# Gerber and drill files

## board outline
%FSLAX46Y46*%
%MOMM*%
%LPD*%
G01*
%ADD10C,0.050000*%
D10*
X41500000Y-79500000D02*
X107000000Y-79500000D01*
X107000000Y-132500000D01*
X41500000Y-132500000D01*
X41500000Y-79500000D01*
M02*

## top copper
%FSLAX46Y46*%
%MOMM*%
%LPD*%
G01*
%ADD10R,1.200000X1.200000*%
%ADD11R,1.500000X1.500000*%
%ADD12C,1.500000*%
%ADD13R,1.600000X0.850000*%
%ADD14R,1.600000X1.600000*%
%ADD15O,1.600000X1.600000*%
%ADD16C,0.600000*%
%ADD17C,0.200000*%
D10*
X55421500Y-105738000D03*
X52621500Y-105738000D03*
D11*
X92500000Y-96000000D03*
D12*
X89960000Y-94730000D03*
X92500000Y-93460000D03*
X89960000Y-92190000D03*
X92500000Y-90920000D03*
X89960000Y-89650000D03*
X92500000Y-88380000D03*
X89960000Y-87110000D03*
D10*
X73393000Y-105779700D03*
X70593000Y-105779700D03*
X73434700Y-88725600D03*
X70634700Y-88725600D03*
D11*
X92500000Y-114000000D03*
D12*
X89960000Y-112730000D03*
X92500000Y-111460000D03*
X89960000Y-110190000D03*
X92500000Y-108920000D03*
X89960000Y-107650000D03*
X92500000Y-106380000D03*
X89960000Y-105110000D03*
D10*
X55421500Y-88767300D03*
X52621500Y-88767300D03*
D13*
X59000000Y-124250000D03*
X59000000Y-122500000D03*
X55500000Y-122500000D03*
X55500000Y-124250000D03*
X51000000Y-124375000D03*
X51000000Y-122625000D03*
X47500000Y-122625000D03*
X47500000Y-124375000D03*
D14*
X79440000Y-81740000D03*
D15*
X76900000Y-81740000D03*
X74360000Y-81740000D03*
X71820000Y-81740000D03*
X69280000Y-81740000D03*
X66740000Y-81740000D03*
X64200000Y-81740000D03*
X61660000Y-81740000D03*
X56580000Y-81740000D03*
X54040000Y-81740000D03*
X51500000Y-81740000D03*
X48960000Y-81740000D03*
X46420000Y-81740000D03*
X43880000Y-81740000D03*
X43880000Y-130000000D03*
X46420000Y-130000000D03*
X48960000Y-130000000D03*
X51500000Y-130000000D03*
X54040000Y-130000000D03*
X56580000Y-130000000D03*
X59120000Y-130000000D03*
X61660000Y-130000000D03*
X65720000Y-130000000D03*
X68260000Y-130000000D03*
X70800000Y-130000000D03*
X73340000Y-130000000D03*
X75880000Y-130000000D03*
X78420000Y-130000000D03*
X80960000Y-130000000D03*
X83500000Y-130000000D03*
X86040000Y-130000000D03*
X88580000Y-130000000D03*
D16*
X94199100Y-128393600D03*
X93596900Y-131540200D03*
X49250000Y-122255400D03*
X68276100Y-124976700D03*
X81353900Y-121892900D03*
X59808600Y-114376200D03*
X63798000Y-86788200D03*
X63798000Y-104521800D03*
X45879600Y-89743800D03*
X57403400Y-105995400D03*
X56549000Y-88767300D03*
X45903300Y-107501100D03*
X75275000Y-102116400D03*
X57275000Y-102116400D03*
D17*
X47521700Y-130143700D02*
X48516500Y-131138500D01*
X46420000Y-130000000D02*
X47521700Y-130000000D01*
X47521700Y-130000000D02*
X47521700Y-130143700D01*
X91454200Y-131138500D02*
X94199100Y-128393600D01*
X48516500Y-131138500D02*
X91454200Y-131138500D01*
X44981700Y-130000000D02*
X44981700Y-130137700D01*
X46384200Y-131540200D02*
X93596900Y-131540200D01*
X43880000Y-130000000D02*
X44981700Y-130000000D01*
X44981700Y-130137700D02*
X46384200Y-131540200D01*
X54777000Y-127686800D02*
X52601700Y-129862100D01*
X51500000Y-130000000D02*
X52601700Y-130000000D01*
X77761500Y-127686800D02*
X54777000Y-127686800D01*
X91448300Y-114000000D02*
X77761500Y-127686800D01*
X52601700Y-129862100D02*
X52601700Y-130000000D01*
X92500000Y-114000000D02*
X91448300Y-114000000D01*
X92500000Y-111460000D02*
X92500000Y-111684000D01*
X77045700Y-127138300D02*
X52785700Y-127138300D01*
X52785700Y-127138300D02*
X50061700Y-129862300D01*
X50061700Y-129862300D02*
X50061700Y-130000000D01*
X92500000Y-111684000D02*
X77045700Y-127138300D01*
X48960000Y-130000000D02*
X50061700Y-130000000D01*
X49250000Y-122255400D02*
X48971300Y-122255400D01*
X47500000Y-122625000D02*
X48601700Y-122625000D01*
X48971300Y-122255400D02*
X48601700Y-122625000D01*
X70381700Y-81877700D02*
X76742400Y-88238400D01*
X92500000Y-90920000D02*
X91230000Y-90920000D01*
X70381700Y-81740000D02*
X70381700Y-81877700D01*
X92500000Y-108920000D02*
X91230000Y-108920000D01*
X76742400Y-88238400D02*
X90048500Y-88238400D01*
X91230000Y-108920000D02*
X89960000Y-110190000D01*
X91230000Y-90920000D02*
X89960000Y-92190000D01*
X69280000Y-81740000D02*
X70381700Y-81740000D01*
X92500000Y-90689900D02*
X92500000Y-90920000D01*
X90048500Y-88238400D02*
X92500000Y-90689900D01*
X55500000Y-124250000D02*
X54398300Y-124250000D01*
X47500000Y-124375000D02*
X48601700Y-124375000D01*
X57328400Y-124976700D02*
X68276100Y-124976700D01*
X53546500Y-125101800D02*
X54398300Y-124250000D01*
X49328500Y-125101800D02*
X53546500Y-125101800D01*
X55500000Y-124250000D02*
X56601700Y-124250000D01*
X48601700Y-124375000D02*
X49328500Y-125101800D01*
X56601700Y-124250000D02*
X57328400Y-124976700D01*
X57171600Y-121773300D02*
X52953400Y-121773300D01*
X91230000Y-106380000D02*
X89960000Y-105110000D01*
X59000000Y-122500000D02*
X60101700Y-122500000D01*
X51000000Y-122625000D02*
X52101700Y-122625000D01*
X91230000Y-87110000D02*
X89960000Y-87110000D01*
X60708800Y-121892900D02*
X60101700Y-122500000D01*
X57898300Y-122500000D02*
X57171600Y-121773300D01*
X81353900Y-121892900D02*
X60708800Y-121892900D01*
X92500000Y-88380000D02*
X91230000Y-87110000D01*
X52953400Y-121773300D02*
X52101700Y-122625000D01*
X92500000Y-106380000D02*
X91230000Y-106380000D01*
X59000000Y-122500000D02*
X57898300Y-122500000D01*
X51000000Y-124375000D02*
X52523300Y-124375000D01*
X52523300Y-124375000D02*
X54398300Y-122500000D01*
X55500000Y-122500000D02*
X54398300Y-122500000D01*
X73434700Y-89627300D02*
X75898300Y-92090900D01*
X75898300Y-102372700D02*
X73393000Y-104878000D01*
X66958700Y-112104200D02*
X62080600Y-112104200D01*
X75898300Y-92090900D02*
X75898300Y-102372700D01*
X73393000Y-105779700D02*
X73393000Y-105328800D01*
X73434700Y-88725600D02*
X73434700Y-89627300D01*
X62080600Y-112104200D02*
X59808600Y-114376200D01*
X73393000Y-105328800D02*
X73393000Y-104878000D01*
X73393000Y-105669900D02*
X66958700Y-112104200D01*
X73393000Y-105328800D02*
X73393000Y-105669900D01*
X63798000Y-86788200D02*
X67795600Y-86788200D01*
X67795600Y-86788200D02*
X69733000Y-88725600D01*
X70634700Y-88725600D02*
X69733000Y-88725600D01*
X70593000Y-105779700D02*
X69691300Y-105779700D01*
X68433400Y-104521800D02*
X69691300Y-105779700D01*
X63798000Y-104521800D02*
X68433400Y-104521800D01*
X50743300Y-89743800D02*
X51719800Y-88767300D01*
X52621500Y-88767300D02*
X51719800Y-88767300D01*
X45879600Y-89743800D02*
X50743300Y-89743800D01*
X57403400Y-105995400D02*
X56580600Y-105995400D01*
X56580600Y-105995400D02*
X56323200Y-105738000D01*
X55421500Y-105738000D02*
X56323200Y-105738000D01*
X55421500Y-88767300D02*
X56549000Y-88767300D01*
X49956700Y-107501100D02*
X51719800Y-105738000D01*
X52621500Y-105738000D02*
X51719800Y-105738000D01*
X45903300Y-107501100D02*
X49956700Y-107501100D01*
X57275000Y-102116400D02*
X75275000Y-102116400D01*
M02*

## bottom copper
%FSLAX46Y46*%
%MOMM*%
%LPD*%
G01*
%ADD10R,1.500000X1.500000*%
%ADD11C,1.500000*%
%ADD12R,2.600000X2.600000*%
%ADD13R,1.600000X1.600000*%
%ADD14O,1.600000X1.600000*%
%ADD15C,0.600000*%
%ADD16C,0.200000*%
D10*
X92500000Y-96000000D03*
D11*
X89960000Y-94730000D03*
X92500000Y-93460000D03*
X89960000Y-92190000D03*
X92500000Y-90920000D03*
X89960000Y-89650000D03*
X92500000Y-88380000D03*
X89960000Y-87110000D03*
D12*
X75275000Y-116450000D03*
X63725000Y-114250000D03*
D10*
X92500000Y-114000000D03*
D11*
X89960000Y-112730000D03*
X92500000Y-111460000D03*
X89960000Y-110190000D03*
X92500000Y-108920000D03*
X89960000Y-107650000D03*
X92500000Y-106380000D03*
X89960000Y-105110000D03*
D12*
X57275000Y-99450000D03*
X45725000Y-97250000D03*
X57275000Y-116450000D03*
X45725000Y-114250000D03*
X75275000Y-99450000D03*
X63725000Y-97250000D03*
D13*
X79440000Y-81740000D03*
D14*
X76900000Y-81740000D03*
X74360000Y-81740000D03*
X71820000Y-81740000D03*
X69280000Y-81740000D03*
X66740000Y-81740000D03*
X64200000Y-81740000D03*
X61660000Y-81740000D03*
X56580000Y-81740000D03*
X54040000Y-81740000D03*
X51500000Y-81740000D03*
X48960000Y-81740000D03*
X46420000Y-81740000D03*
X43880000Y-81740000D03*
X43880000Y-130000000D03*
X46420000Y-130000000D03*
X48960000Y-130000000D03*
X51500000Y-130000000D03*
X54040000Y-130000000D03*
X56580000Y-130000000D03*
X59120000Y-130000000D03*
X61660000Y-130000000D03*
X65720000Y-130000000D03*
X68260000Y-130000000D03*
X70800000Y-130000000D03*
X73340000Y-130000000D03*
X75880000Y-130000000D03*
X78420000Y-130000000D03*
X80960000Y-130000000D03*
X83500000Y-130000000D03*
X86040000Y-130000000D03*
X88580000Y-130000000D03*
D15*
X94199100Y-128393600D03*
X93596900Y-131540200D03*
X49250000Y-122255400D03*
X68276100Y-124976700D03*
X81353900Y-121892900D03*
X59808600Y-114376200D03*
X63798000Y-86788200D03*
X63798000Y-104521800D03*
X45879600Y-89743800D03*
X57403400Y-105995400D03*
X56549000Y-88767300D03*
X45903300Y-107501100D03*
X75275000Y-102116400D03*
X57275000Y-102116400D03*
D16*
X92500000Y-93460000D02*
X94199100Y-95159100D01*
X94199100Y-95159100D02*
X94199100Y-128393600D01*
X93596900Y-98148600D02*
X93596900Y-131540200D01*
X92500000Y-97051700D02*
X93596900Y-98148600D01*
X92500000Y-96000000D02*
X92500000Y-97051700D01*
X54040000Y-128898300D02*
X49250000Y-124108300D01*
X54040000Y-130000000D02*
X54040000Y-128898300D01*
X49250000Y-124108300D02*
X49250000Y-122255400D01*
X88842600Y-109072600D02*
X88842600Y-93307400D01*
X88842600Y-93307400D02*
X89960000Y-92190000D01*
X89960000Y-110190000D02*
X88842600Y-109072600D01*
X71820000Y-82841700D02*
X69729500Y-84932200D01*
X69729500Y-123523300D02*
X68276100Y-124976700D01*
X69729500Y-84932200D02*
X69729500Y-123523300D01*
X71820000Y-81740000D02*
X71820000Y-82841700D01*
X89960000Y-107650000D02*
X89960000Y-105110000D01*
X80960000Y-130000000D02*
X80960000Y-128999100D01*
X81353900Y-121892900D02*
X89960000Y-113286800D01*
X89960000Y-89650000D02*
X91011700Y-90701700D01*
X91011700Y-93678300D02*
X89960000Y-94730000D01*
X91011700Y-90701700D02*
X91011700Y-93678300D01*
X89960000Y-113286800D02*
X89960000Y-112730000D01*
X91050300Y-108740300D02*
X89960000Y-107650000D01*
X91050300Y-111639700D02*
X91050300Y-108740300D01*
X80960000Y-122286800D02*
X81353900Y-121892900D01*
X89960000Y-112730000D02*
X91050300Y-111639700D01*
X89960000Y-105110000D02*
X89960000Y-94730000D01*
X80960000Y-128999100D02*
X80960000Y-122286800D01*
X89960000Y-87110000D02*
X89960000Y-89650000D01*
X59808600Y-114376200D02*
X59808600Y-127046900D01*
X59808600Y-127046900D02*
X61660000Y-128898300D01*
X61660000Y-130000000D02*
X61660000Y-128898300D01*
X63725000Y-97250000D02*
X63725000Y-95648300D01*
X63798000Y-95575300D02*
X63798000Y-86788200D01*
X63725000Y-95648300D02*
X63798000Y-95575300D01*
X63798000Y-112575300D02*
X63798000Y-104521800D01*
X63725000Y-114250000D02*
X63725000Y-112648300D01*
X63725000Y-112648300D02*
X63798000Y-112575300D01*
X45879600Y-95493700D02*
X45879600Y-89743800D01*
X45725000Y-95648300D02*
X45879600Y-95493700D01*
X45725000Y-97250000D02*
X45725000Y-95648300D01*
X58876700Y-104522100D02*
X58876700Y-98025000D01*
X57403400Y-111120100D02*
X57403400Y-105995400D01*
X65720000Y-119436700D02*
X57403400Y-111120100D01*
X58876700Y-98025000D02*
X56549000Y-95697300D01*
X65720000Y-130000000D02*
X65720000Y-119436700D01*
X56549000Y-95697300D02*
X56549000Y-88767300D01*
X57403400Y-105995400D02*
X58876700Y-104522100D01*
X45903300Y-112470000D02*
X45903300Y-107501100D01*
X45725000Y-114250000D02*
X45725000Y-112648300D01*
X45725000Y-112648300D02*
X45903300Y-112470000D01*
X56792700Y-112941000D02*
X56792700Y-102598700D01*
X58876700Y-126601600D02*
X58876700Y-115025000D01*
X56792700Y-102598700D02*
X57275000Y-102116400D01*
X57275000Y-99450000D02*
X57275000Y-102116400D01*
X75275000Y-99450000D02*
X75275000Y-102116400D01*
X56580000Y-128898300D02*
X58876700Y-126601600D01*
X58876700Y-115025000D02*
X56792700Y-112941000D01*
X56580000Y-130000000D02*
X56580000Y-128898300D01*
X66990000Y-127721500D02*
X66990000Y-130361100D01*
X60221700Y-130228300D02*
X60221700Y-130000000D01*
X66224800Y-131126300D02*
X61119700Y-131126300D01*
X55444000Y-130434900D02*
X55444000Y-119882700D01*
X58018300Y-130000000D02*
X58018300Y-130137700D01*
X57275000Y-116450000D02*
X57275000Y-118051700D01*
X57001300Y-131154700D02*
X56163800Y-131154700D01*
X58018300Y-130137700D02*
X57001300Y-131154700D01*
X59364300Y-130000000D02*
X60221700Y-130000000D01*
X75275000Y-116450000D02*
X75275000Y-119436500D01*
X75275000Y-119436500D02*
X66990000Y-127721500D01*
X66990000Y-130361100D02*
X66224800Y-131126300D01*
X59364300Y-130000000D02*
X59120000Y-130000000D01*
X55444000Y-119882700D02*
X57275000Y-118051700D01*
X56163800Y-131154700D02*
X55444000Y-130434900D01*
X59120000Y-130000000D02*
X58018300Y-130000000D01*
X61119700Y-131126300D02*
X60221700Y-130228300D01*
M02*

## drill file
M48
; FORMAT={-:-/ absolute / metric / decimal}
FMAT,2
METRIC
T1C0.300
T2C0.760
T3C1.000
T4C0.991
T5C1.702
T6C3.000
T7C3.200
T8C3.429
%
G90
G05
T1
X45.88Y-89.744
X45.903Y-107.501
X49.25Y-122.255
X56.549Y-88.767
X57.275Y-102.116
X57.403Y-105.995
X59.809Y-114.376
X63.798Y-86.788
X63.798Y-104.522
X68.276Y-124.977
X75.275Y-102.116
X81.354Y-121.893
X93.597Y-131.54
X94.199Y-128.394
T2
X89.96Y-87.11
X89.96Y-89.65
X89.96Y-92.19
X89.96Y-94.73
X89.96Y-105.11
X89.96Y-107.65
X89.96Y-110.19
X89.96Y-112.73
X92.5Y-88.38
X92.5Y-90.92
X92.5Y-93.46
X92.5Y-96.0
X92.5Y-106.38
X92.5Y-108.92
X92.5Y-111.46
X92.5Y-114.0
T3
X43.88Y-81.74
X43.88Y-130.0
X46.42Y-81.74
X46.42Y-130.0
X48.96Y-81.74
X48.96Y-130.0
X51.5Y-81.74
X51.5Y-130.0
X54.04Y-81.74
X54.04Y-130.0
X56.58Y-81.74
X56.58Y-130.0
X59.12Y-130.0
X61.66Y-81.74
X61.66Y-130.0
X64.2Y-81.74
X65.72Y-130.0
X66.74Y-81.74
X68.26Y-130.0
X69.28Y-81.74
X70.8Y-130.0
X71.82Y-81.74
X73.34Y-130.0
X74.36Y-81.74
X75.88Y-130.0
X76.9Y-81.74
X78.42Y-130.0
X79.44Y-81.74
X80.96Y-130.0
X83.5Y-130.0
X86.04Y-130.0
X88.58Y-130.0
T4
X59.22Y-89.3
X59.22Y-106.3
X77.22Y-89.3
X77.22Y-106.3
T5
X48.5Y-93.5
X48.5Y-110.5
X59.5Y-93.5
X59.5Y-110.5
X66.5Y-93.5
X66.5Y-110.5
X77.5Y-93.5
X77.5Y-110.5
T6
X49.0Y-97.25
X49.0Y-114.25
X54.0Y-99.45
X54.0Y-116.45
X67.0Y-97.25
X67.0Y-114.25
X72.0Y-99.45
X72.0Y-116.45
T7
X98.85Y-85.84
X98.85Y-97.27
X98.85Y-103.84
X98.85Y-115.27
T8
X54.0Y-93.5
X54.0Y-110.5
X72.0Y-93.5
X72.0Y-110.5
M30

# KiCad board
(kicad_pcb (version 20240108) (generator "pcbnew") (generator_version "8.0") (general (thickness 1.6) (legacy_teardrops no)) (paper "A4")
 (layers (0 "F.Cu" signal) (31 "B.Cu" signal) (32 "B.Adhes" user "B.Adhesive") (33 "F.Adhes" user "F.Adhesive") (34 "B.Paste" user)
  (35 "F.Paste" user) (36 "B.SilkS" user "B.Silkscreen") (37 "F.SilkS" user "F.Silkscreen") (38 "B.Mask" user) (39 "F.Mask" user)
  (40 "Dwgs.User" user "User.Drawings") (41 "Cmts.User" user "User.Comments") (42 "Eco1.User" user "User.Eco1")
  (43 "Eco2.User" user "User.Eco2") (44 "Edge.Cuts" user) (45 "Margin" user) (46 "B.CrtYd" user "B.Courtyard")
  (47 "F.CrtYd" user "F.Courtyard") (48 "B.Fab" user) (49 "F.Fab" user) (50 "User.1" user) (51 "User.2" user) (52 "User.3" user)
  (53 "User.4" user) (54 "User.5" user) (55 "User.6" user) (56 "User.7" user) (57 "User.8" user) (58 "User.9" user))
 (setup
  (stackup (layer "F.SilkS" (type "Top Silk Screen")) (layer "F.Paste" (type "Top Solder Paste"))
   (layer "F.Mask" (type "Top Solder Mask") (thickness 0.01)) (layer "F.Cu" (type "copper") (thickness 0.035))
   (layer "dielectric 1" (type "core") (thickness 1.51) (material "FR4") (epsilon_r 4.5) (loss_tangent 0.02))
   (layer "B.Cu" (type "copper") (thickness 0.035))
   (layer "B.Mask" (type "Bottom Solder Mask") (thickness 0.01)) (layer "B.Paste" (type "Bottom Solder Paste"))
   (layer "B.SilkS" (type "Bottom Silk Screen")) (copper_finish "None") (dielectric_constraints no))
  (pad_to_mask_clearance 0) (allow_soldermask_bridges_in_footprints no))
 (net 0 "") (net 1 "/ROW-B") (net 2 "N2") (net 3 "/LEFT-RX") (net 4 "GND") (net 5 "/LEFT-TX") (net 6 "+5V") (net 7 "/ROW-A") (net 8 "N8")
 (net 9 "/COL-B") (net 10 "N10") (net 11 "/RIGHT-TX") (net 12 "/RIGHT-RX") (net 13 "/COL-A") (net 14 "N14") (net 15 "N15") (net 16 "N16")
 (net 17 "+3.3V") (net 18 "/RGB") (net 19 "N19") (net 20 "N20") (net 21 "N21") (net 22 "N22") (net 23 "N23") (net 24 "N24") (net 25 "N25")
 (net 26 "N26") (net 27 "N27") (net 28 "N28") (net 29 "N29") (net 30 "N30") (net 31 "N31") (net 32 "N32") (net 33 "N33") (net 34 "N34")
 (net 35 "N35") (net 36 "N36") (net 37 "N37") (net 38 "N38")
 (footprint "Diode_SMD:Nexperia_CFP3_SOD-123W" (layer "F.Cu") (at 54.0215 105.738 180)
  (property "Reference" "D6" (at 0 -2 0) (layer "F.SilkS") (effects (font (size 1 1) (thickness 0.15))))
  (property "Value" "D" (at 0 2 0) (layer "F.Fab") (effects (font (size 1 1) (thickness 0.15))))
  (pad "1" smd rect (at -1.4 0 180) (size 1.2 1.2) (layers "F.Cu" "F.Paste" "F.Mask") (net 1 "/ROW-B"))
  (pad "2" smd rect (at 1.4 0 180) (size 1.2 1.2) (layers "F.Cu" "F.Paste" "F.Mask") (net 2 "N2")))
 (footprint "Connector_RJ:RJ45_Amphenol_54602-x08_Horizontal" (layer "F.Cu") (at 92.5 96 90)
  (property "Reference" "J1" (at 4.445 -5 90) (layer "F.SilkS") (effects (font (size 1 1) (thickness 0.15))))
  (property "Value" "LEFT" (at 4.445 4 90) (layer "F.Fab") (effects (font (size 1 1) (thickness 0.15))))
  (pad "" np_thru_hole circle (at -1.27 6.35 90) (size 3.2 3.2) (drill 3.2) (layers "*.Cu" "*.Mask"))
  (pad "" np_thru_hole circle (at 10.16 6.35 90) (size 3.2 3.2) (drill 3.2) (layers "*.Cu" "*.Mask"))
  (pad "1" thru_hole rect (at 0 0 90) (size 1.5 1.5) (drill 0.76) (layers "*.Cu" "*.Mask") (remove_unused_layers no) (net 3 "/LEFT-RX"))
  (pad "2" thru_hole circle (at 1.27 -2.54 90) (size 1.5 1.5) (drill 0.76) (layers "*.Cu" "*.Mask") (remove_unused_layers no) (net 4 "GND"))
  (pad "3" thru_hole circle (at 2.54 0 90) (size 1.5 1.5) (drill 0.76) (layers "*.Cu" "*.Mask") (remove_unused_layers no) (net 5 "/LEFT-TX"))
  (pad "4" thru_hole circle (at 3.81 -2.54 90) (size 1.5 1.5) (drill 0.76) (layers "*.Cu" "*.Mask") (remove_unused_layers no) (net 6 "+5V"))
  (pad "5" thru_hole circle (at 5.08 0 90) (size 1.5 1.5) (drill 0.76) (layers "*.Cu" "*.Mask") (remove_unused_layers no) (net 6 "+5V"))
  (pad "6" thru_hole circle (at 6.35 -2.54 90) (size 1.5 1.5) (drill 0.76) (layers "*.Cu" "*.Mask") (remove_unused_layers no) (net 4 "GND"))
  (pad "7" thru_hole circle (at 7.62 0 90) (size 1.5 1.5) (drill 0.76) (layers "*.Cu" "*.Mask") (remove_unused_layers no) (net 4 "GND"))
  (pad "8" thru_hole circle (at 8.89 -2.54 90) (size 1.5 1.5) (drill 0.76) (layers "*.Cu" "*.Mask") (remove_unused_layers no) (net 4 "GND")))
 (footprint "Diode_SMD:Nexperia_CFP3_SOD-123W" (layer "F.Cu") (at 71.993 105.7797 180)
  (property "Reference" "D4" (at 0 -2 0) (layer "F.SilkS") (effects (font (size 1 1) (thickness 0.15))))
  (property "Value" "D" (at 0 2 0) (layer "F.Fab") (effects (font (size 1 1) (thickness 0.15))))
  (pad "1" smd rect (at -1.4 0 180) (size 1.2 1.2) (layers "F.Cu" "F.Paste" "F.Mask") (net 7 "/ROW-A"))
  (pad "2" smd rect (at 1.4 0 180) (size 1.2 1.2) (layers "F.Cu" "F.Paste" "F.Mask") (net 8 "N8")))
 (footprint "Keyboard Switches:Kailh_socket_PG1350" (layer "F.Cu") (at 72 110.5)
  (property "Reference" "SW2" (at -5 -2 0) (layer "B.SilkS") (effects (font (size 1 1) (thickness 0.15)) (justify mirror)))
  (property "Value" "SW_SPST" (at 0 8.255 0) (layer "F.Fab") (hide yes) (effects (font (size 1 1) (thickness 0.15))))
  (pad "" np_thru_hole circle (at -5.5 0) (size 1.7018 1.7018) (drill 1.7018) (layers "*.Cu" "*.Mask"))
  (pad "" np_thru_hole circle (at -5 3.75) (size 3 3) (drill 3) (layers "*.Cu" "*.Mask"))
  (pad "" np_thru_hole circle (at 0 0) (size 3.429 3.429) (drill 3.429) (layers "*.Cu" "*.Mask"))
  (pad "" np_thru_hole circle (at 0 5.95) (size 3 3) (drill 3) (layers "*.Cu" "*.Mask"))
  (pad "" np_thru_hole circle (at 5.22 -4.2) (size 0.9906 0.9906) (drill 0.9906) (layers "*.Cu" "*.Mask"))
  (pad "" np_thru_hole circle (at 5.5 0) (size 1.7018 1.7018) (drill 1.7018) (layers "*.Cu" "*.Mask"))
  (pad "1" smd rect (at 3.275 5.95) (size 2.6 2.6) (layers "B.Cu" "B.Paste" "B.Mask") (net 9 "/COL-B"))
  (pad "2" smd rect (at -8.275 3.75) (size 2.6 2.6) (layers "B.Cu" "B.Paste" "B.Mask") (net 8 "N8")))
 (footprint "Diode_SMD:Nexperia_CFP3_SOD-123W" (layer "F.Cu") (at 72.0347 88.7256 180)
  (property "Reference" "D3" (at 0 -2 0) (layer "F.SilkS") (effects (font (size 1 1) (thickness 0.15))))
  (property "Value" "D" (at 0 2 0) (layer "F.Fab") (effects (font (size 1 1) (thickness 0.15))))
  (pad "1" smd rect (at -1.4 0 180) (size 1.2 1.2) (layers "F.Cu" "F.Paste" "F.Mask") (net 7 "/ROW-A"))
  (pad "2" smd rect (at 1.4 0 180) (size 1.2 1.2) (layers "F.Cu" "F.Paste" "F.Mask") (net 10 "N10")))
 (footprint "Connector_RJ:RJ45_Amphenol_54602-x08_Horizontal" (layer "F.Cu") (at 92.5 114 90)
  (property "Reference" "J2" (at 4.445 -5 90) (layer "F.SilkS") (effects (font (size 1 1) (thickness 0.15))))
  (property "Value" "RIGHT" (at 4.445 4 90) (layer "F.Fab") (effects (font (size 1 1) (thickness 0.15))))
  (pad "" np_thru_hole circle (at -1.27 6.35 90) (size 3.2 3.2) (drill 3.2) (layers "*.Cu" "*.Mask"))
  (pad "" np_thru_hole circle (at 10.16 6.35 90) (size 3.2 3.2) (drill 3.2) (layers "*.Cu" "*.Mask"))
  (pad "1" thru_hole rect (at 0 0 90) (size 1.5 1.5) (drill 0.76) (layers "*.Cu" "*.Mask") (remove_unused_layers no) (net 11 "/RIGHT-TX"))
  (pad "2" thru_hole circle (at 1.27 -2.54 90) (size 1.5 1.5) (drill 0.76) (layers "*.Cu" "*.Mask") (remove_unused_layers no) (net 4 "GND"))
  (pad "3" thru_hole circle (at 2.54 0 90) (size 1.5 1.5) (drill 0.76) (layers "*.Cu" "*.Mask") (remove_unused_layers no)
   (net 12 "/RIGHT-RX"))
  (pad "4" thru_hole circle (at 3.81 -2.54 90) (size 1.5 1.5) (drill 0.76) (layers "*.Cu" "*.Mask") (remove_unused_layers no) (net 6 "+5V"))
  (pad "5" thru_hole circle (at 5.08 0 90) (size 1.5 1.5) (drill 0.76) (layers "*.Cu" "*.Mask") (remove_unused_layers no) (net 6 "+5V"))
  (pad "6" thru_hole circle (at 6.35 -2.54 90) (size 1.5 1.5) (drill 0.76) (layers "*.Cu" "*.Mask") (remove_unused_layers no) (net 4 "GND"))
  (pad "7" thru_hole circle (at 7.62 0 90) (size 1.5 1.5) (drill 0.76) (layers "*.Cu" "*.Mask") (remove_unused_layers no) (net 4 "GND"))
  (pad "8" thru_hole circle (at 8.89 -2.54 90) (size 1.5 1.5) (drill 0.76) (layers "*.Cu" "*.Mask") (remove_unused_layers no) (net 4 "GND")))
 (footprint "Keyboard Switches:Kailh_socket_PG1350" (layer "F.Cu") (at 54 93.5)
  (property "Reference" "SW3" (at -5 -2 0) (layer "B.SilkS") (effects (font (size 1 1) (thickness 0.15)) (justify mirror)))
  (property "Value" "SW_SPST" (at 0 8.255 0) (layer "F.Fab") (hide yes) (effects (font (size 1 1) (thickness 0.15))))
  (pad "" np_thru_hole circle (at -5.5 0) (size 1.7018 1.7018) (drill 1.7018) (layers "*.Cu" "*.Mask"))
  (pad "" np_thru_hole circle (at -5 3.75) (size 3 3) (drill 3) (layers "*.Cu" "*.Mask"))
  (pad "" np_thru_hole circle (at 0 0) (size 3.429 3.429) (drill 3.429) (layers "*.Cu" "*.Mask"))
  (pad "" np_thru_hole circle (at 0 5.95) (size 3 3) (drill 3) (layers "*.Cu" "*.Mask"))
  (pad "" np_thru_hole circle (at 5.22 -4.2) (size 0.9906 0.9906) (drill 0.9906) (layers "*.Cu" "*.Mask"))
  (pad "" np_thru_hole circle (at 5.5 0) (size 1.7018 1.7018) (drill 1.7018) (layers "*.Cu" "*.Mask"))
  (pad "1" smd rect (at 3.275 5.95) (size 2.6 2.6) (layers "B.Cu" "B.Paste" "B.Mask") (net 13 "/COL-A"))
  (pad "2" smd rect (at -8.275 3.75) (size 2.6 2.6) (layers "B.Cu" "B.Paste" "B.Mask") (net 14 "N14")))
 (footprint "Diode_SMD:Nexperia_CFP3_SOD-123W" (layer "F.Cu") (at 54.0215 88.7673 180)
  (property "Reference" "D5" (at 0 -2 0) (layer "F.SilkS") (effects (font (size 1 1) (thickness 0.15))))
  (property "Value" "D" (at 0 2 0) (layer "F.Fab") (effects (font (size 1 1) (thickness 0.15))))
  (pad "1" smd rect (at -1.4 0 180) (size 1.2 1.2) (layers "F.Cu" "F.Paste" "F.Mask") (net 1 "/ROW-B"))
  (pad "2" smd rect (at 1.4 0 180) (size 1.2 1.2) (layers "F.Cu" "F.Paste" "F.Mask") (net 14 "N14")))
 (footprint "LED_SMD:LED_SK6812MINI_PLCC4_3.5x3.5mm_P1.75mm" (layer "F.Cu") (at 57.25 123.375 180)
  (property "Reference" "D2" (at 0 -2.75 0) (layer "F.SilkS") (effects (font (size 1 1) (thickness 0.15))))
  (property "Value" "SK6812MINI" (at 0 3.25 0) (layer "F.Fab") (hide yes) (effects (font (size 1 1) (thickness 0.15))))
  (pad "1" smd rect (at -1.75 -0.875 180) (size 1.6 0.85) (layers "F.Cu" "F.Paste" "F.Mask") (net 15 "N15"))
  (pad "2" smd rect (at -1.75 0.875 180) (size 1.6 0.85) (layers "F.Cu" "F.Paste" "F.Mask") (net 4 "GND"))
  (pad "3" smd rect (at 1.75 0.875 180) (size 1.6 0.85) (layers "F.Cu" "F.Paste" "F.Mask") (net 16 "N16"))
  (pad "4" smd rect (at 1.75 -0.875 180) (size 1.6 0.85) (layers "F.Cu" "F.Paste" "F.Mask") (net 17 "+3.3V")))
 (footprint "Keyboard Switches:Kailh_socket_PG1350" (layer "F.Cu") (at 54 110.5)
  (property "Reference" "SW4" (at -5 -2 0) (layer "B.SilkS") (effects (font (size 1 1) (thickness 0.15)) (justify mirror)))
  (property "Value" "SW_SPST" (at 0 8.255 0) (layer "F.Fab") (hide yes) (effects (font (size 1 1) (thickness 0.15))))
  (pad "" np_thru_hole circle (at -5.5 0) (size 1.7018 1.7018) (drill 1.7018) (layers "*.Cu" "*.Mask"))
  (pad "" np_thru_hole circle (at -5 3.75) (size 3 3) (drill 3) (layers "*.Cu" "*.Mask"))
  (pad "" np_thru_hole circle (at 0 0) (size 3.429 3.429) (drill 3.429) (layers "*.Cu" "*.Mask"))
  (pad "" np_thru_hole circle (at 0 5.95) (size 3 3) (drill 3) (layers "*.Cu" "*.Mask"))
  (pad "" np_thru_hole circle (at 5.22 -4.2) (size 0.9906 0.9906) (drill 0.9906) (layers "*.Cu" "*.Mask"))
  (pad "" np_thru_hole circle (at 5.5 0) (size 1.7018 1.7018) (drill 1.7018) (layers "*.Cu" "*.Mask"))
  (pad "1" smd rect (at 3.275 5.95) (size 2.6 2.6) (layers "B.Cu" "B.Paste" "B.Mask") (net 9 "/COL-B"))
  (pad "2" smd rect (at -8.275 3.75) (size 2.6 2.6) (layers "B.Cu" "B.Paste" "B.Mask") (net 2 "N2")))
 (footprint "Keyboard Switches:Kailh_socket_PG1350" (layer "F.Cu") (at 72 93.5)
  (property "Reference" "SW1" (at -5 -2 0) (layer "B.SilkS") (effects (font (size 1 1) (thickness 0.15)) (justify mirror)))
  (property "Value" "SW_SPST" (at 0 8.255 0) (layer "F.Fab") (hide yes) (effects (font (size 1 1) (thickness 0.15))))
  (pad "" np_thru_hole circle (at -5.5 0) (size 1.7018 1.7018) (drill 1.7018) (layers "*.Cu" "*.Mask"))
  (pad "" np_thru_hole circle (at -5 3.75) (size 3 3) (drill 3) (layers "*.Cu" "*.Mask"))
  (pad "" np_thru_hole circle (at 0 0) (size 3.429 3.429) (drill 3.429) (layers "*.Cu" "*.Mask"))
  (pad "" np_thru_hole circle (at 0 5.95) (size 3 3) (drill 3) (layers "*.Cu" "*.Mask"))
  (pad "" np_thru_hole circle (at 5.22 -4.2) (size 0.9906 0.9906) (drill 0.9906) (layers "*.Cu" "*.Mask"))
  (pad "" np_thru_hole circle (at 5.5 0) (size 1.7018 1.7018) (drill 1.7018) (layers "*.Cu" "*.Mask"))
  (pad "1" smd rect (at 3.275 5.95) (size 2.6 2.6) (layers "B.Cu" "B.Paste" "B.Mask") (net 13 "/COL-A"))
  (pad "2" smd rect (at -8.275 3.75) (size 2.6 2.6) (layers "B.Cu" "B.Paste" "B.Mask") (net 10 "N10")))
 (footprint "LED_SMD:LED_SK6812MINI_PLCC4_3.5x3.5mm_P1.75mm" (layer "F.Cu") (at 49.25 123.5 180)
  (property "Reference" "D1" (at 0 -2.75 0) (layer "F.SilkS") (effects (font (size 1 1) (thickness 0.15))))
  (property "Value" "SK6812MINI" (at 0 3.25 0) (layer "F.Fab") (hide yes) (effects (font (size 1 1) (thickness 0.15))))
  (pad "1" smd rect (at -1.75 -0.875 180) (size 1.6 0.85) (layers "F.Cu" "F.Paste" "F.Mask") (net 16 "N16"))
  (pad "2" smd rect (at -1.75 0.875 180) (size 1.6 0.85) (layers "F.Cu" "F.Paste" "F.Mask") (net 4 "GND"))
  (pad "3" smd rect (at 1.75 0.875 180) (size 1.6 0.85) (layers "F.Cu" "F.Paste" "F.Mask") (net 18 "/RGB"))
  (pad "4" smd rect (at 1.75 -0.875 180) (size 1.6 0.85) (layers "F.Cu" "F.Paste" "F.Mask") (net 17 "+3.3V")))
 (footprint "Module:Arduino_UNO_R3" (layer "B.Cu") (at 79.44 81.74 180)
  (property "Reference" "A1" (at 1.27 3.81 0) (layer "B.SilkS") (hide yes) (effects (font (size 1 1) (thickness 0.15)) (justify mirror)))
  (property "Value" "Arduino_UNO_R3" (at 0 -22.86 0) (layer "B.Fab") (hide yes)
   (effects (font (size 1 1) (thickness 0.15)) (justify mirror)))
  (pad "1" thru_hole rect (at 0 0 90) (size 1.6 1.6) (drill 1) (layers "*.Cu" "*.Mask") (remove_unused_layers no) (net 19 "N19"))
  (pad "2" thru_hole oval (at 2.54 0 90) (size 1.6 1.6) (drill 1) (layers "*.Cu" "*.Mask") (remove_unused_layers no) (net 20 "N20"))
  (pad "3" thru_hole oval (at 5.08 0 90) (size 1.6 1.6) (drill 1) (layers "*.Cu" "*.Mask") (remove_unused_layers no) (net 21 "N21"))
  (pad "4" thru_hole oval (at 7.62 0 90) (size 1.6 1.6) (drill 1) (layers "*.Cu" "*.Mask") (remove_unused_layers no) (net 17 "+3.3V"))
  (pad "5" thru_hole oval (at 10.16 0 90) (size 1.6 1.6) (drill 1) (layers "*.Cu" "*.Mask") (remove_unused_layers no) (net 6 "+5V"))
  (pad "6" thru_hole oval (at 12.7 0 90) (size 1.6 1.6) (drill 1) (layers "*.Cu" "*.Mask") (remove_unused_layers no) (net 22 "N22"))
  (pad "7" thru_hole oval (at 15.24 0 90) (size 1.6 1.6) (drill 1) (layers "*.Cu" "*.Mask") (remove_unused_layers no) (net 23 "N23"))
  (pad "8" thru_hole oval (at 17.78 0 90) (size 1.6 1.6) (drill 1) (layers "*.Cu" "*.Mask") (remove_unused_layers no) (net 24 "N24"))
  (pad "9" thru_hole oval (at 22.86 0 90) (size 1.6 1.6) (drill 1) (layers "*.Cu" "*.Mask") (remove_unused_layers no) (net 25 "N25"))
  (pad "10" thru_hole oval (at 25.4 0 90) (size 1.6 1.6) (drill 1) (layers "*.Cu" "*.Mask") (remove_unused_layers no) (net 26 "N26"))
  (pad "11" thru_hole oval (at 27.94 0 90) (size 1.6 1.6) (drill 1) (layers "*.Cu" "*.Mask") (remove_unused_layers no) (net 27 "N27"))
  (pad "12" thru_hole oval (at 30.48 0 90) (size 1.6 1.6) (drill 1) (layers "*.Cu" "*.Mask") (remove_unused_layers no) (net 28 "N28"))
  (pad "13" thru_hole oval (at 33.02 0 90) (size 1.6 1.6) (drill 1) (layers "*.Cu" "*.Mask") (remove_unused_layers no) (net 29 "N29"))
  (pad "14" thru_hole oval (at 35.56 0 90) (size 1.6 1.6) (drill 1) (layers "*.Cu" "*.Mask") (remove_unused_layers no) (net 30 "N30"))
  (pad "15" thru_hole oval (at 35.56 -48.26 90) (size 1.6 1.6) (drill 1) (layers "*.Cu" "*.Mask") (remove_unused_layers no)
   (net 3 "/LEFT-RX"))
  (pad "16" thru_hole oval (at 33.02 -48.26 90) (size 1.6 1.6) (drill 1) (layers "*.Cu" "*.Mask") (remove_unused_layers no)
   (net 5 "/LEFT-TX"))
  (pad "17" thru_hole oval (at 30.48 -48.26 90) (size 1.6 1.6) (drill 1) (layers "*.Cu" "*.Mask") (remove_unused_layers no)
   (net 12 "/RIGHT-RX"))
  (pad "18" thru_hole oval (at 27.94 -48.26 90) (size 1.6 1.6) (drill 1) (layers "*.Cu" "*.Mask") (remove_unused_layers no)
   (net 11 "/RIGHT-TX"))
  (pad "19" thru_hole oval (at 25.4 -48.26 90) (size 1.6 1.6) (drill 1) (layers "*.Cu" "*.Mask") (remove_unused_layers no) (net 18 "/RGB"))
  (pad "20" thru_hole oval (at 22.86 -48.26 90) (size 1.6 1.6) (drill 1) (layers "*.Cu" "*.Mask") (remove_unused_layers no)
   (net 13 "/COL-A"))
  (pad "21" thru_hole oval (at 20.32 -48.26 90) (size 1.6 1.6) (drill 1) (layers "*.Cu" "*.Mask") (remove_unused_layers no) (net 9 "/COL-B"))
  (pad "22" thru_hole oval (at 17.78 -48.26 90) (size 1.6 1.6) (drill 1) (layers "*.Cu" "*.Mask") (remove_unused_layers no) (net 7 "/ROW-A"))
  (pad "23" thru_hole oval (at 13.72 -48.26 90) (size 1.6 1.6) (drill 1) (layers "*.Cu" "*.Mask") (remove_unused_layers no) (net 1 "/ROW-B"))
  (pad "24" thru_hole oval (at 11.18 -48.26 90) (size 1.6 1.6) (drill 1) (layers "*.Cu" "*.Mask") (remove_unused_layers no) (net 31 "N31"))
  (pad "25" thru_hole oval (at 8.64 -48.26 90) (size 1.6 1.6) (drill 1) (layers "*.Cu" "*.Mask") (remove_unused_layers no) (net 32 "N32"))
  (pad "26" thru_hole oval (at 6.1 -48.26 90) (size 1.6 1.6) (drill 1) (layers "*.Cu" "*.Mask") (remove_unused_layers no) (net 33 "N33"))
  (pad "27" thru_hole oval (at 3.56 -48.26 90) (size 1.6 1.6) (drill 1) (layers "*.Cu" "*.Mask") (remove_unused_layers no) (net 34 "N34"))
  (pad "28" thru_hole oval (at 1.02 -48.26 90) (size 1.6 1.6) (drill 1) (layers "*.Cu" "*.Mask") (remove_unused_layers no) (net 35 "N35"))
  (pad "29" thru_hole oval (at -1.52 -48.26 90) (size 1.6 1.6) (drill 1) (layers "*.Cu" "*.Mask") (remove_unused_layers no) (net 4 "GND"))
  (pad "30" thru_hole oval (at -4.06 -48.26 90) (size 1.6 1.6) (drill 1) (layers "*.Cu" "*.Mask") (remove_unused_layers no) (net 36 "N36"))
  (pad "31" thru_hole oval (at -6.6 -48.26 90) (size 1.6 1.6) (drill 1) (layers "*.Cu" "*.Mask") (remove_unused_layers no) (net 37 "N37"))
  (pad "32" thru_hole oval (at -9.14 -48.26 90) (size 1.6 1.6) (drill 1) (layers "*.Cu" "*.Mask") (remove_unused_layers no) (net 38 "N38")))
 (gr_rect (start 41.5 79.5) (end 107 132.5) (stroke (width 0.05) (type default)) (fill none) (layer "Edge.Cuts"))
 (segment (start 47.5217 130.1437) (end 48.5165 131.1385) (width 0.2) (layer "F.Cu") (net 5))
 (segment (start 46.42 130) (end 47.5217 130) (width 0.2) (layer "F.Cu") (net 5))
 (segment (start 47.5217 130) (end 47.5217 130.1437) (width 0.2) (layer "F.Cu") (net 5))
 (segment (start 91.4542 131.1385) (end 94.1991 128.3936) (width 0.2) (layer "F.Cu") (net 5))
 (segment (start 48.5165 131.1385) (end 91.4542 131.1385) (width 0.2) (layer "F.Cu") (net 5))
 (via (at 94.1991 128.3936) (size 0.6) (drill 0.3) (layers "F.Cu" "B.Cu") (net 5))
 (segment (start 92.5 93.46) (end 94.1991 95.1591) (width 0.2) (layer "B.Cu") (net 5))
 (segment (start 94.1991 95.1591) (end 94.1991 128.3936) (width 0.2) (layer "B.Cu") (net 5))
 (segment (start 44.9817 130) (end 44.9817 130.1377) (width 0.2) (layer "F.Cu") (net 3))
 (segment (start 46.3842 131.5402) (end 93.5969 131.5402) (width 0.2) (layer "F.Cu") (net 3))
 (segment (start 43.88 130) (end 44.9817 130) (width 0.2) (layer "F.Cu") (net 3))
 (segment (start 44.9817 130.1377) (end 46.3842 131.5402) (width 0.2) (layer "F.Cu") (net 3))
 (via (at 93.5969 131.5402) (size 0.6) (drill 0.3) (layers "F.Cu" "B.Cu") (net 3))
 (segment (start 93.5969 98.1486) (end 93.5969 131.5402) (width 0.2) (layer "B.Cu") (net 3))
 (segment (start 92.5 97.0517) (end 93.5969 98.1486) (width 0.2) (layer "B.Cu") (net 3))
 (segment (start 92.5 96) (end 92.5 97.0517) (width 0.2) (layer "B.Cu") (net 3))
 (segment (start 54.777 127.6868) (end 52.6017 129.8621) (width 0.2) (layer "F.Cu") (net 11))
 (segment (start 51.5 130) (end 52.6017 130) (width 0.2) (layer "F.Cu") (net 11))
 (segment (start 77.7615 127.6868) (end 54.777 127.6868) (width 0.2) (layer "F.Cu") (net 11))
 (segment (start 91.4483 114) (end 77.7615 127.6868) (width 0.2) (layer "F.Cu") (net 11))
 (segment (start 52.6017 129.8621) (end 52.6017 130) (width 0.2) (layer "F.Cu") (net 11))
 (segment (start 92.5 114) (end 91.4483 114) (width 0.2) (layer "F.Cu") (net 11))
 (segment (start 92.5 111.46) (end 92.5 111.684) (width 0.2) (layer "F.Cu") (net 12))
 (segment (start 77.0457 127.1383) (end 52.7857 127.1383) (width 0.2) (layer "F.Cu") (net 12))
 (segment (start 52.7857 127.1383) (end 50.0617 129.8623) (width 0.2) (layer "F.Cu") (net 12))
 (segment (start 50.0617 129.8623) (end 50.0617 130) (width 0.2) (layer "F.Cu") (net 12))
 (segment (start 92.5 111.684) (end 77.0457 127.1383) (width 0.2) (layer "F.Cu") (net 12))
 (segment (start 48.96 130) (end 50.0617 130) (width 0.2) (layer "F.Cu") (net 12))
 (segment (start 49.25 122.2554) (end 48.9713 122.2554) (width 0.2) (layer "F.Cu") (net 18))
 (segment (start 47.5 122.625) (end 48.6017 122.625) (width 0.2) (layer "F.Cu") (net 18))
 (segment (start 48.9713 122.2554) (end 48.6017 122.625) (width 0.2) (layer "F.Cu") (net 18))
 (via (at 49.25 122.2554) (size 0.6) (drill 0.3) (layers "F.Cu" "B.Cu") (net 18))
 (segment (start 54.04 128.8983) (end 49.25 124.1083) (width 0.2) (layer "B.Cu") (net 18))
 (segment (start 54.04 130) (end 54.04 128.8983) (width 0.2) (layer "B.Cu") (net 18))
 (segment (start 49.25 124.1083) (end 49.25 122.2554) (width 0.2) (layer "B.Cu") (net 18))
 (segment (start 70.3817 81.8777) (end 76.7424 88.2384) (width 0.2) (layer "F.Cu") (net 6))
 (segment (start 92.5 90.92) (end 91.23 90.92) (width 0.2) (layer "F.Cu") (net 6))
 (segment (start 70.3817 81.74) (end 70.3817 81.8777) (width 0.2) (layer "F.Cu") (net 6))
 (segment (start 92.5 108.92) (end 91.23 108.92) (width 0.2) (layer "F.Cu") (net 6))
 (segment (start 76.7424 88.2384) (end 90.0485 88.2384) (width 0.2) (layer "F.Cu") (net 6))
 (segment (start 91.23 108.92) (end 89.96 110.19) (width 0.2) (layer "F.Cu") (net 6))
 (segment (start 91.23 90.92) (end 89.96 92.19) (width 0.2) (layer "F.Cu") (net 6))
 (segment (start 69.28 81.74) (end 70.3817 81.74) (width 0.2) (layer "F.Cu") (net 6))
 (segment (start 92.5 90.6899) (end 92.5 90.92) (width 0.2) (layer "F.Cu") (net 6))
 (segment (start 90.0485 88.2384) (end 92.5 90.6899) (width 0.2) (layer "F.Cu") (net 6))
 (segment (start 88.8426 109.0726) (end 88.8426 93.3074) (width 0.2) (layer "B.Cu") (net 6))
 (segment (start 88.8426 93.3074) (end 89.96 92.19) (width 0.2) (layer "B.Cu") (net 6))
 (segment (start 89.96 110.19) (end 88.8426 109.0726) (width 0.2) (layer "B.Cu") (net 6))
 (segment (start 55.5 124.25) (end 54.3983 124.25) (width 0.2) (layer "F.Cu") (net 17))
 (segment (start 47.5 124.375) (end 48.6017 124.375) (width 0.2) (layer "F.Cu") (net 17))
 (segment (start 57.3284 124.9767) (end 68.2761 124.9767) (width 0.2) (layer "F.Cu") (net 17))
 (segment (start 53.5465 125.1018) (end 54.3983 124.25) (width 0.2) (layer "F.Cu") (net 17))
 (segment (start 49.3285 125.1018) (end 53.5465 125.1018) (width 0.2) (layer "F.Cu") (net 17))
 (segment (start 55.5 124.25) (end 56.6017 124.25) (width 0.2) (layer "F.Cu") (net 17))
 (segment (start 48.6017 124.375) (end 49.3285 125.1018) (width 0.2) (layer "F.Cu") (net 17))
 (segment (start 56.6017 124.25) (end 57.3284 124.9767) (width 0.2) (layer "F.Cu") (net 17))
 (via (at 68.2761 124.9767) (size 0.6) (drill 0.3) (layers "F.Cu" "B.Cu") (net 17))
 (segment (start 71.82 82.8417) (end 69.7295 84.9322) (width 0.2) (layer "B.Cu") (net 17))
 (segment (start 69.7295 123.5233) (end 68.2761 124.9767) (width 0.2) (layer "B.Cu") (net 17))
 (segment (start 69.7295 84.9322) (end 69.7295 123.5233) (width 0.2) (layer "B.Cu") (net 17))
 (segment (start 71.82 81.74) (end 71.82 82.8417) (width 0.2) (layer "B.Cu") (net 17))
 (segment (start 57.1716 121.7733) (end 52.9534 121.7733) (width 0.2) (layer "F.Cu") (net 4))
 (segment (start 91.23 106.38) (end 89.96 105.11) (width 0.2) (layer "F.Cu") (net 4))
 (segment (start 59 122.5) (end 60.1017 122.5) (width 0.2) (layer "F.Cu") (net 4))
 (segment (start 51 122.625) (end 52.1017 122.625) (width 0.2) (layer "F.Cu") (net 4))
 (segment (start 91.23 87.11) (end 89.96 87.11) (width 0.2) (layer "F.Cu") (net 4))
 (segment (start 60.7088 121.8929) (end 60.1017 122.5) (width 0.2) (layer "F.Cu") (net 4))
 (segment (start 57.8983 122.5) (end 57.1716 121.7733) (width 0.2) (layer "F.Cu") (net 4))
 (segment (start 81.3539 121.8929) (end 60.7088 121.8929) (width 0.2) (layer "F.Cu") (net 4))
 (segment (start 92.5 88.38) (end 91.23 87.11) (width 0.2) (layer "F.Cu") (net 4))
 (segment (start 52.9534 121.7733) (end 52.1017 122.625) (width 0.2) (layer "F.Cu") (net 4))
 (segment (start 92.5 106.38) (end 91.23 106.38) (width 0.2) (layer "F.Cu") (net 4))
 (segment (start 59 122.5) (end 57.8983 122.5) (width 0.2) (layer "F.Cu") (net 4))
 (via (at 81.3539 121.8929) (size 0.6) (drill 0.3) (layers "F.Cu" "B.Cu") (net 4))
 (segment (start 89.96 107.65) (end 89.96 105.11) (width 0.2) (layer "B.Cu") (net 4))
 (segment (start 80.96 130) (end 80.96 128.9991) (width 0.2) (layer "B.Cu") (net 4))
 (segment (start 81.3539 121.8929) (end 89.96 113.2868) (width 0.2) (layer "B.Cu") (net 4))
 (segment (start 89.96 89.65) (end 91.0117 90.7017) (width 0.2) (layer "B.Cu") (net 4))
 (segment (start 91.0117 93.6783) (end 89.96 94.73) (width 0.2) (layer "B.Cu") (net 4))
 (segment (start 91.0117 90.7017) (end 91.0117 93.6783) (width 0.2) (layer "B.Cu") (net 4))
 (segment (start 89.96 113.2868) (end 89.96 112.73) (width 0.2) (layer "B.Cu") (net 4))
 (segment (start 91.0503 108.7403) (end 89.96 107.65) (width 0.2) (layer "B.Cu") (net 4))
 (segment (start 91.0503 111.6397) (end 91.0503 108.7403) (width 0.2) (layer "B.Cu") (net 4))
 (segment (start 80.96 122.2868) (end 81.3539 121.8929) (width 0.2) (layer "B.Cu") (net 4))
 (segment (start 89.96 112.73) (end 91.0503 111.6397) (width 0.2) (layer "B.Cu") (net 4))
 (segment (start 89.96 105.11) (end 89.96 94.73) (width 0.2) (layer "B.Cu") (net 4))
 (segment (start 80.96 128.9991) (end 80.96 122.2868) (width 0.2) (layer "B.Cu") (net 4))
 (segment (start 89.96 87.11) (end 89.96 89.65) (width 0.2) (layer "B.Cu") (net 4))
 (segment (start 51 124.375) (end 52.5233 124.375) (width 0.2) (layer "F.Cu") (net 16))
 (segment (start 52.5233 124.375) (end 54.3983 122.5) (width 0.2) (layer "F.Cu") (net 16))
 (segment (start 55.5 122.5) (end 54.3983 122.5) (width 0.2) (layer "F.Cu") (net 16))
 (segment (start 73.4347 89.6273) (end 75.8983 92.0909) (width 0.2) (layer "F.Cu") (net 7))
 (segment (start 75.8983 102.3727) (end 73.393 104.878) (width 0.2) (layer "F.Cu") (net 7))
 (segment (start 66.9587 112.1042) (end 62.0806 112.1042) (width 0.2) (layer "F.Cu") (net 7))
 (segment (start 75.8983 92.0909) (end 75.8983 102.3727) (width 0.2) (layer "F.Cu") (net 7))
 (segment (start 73.393 105.7797) (end 73.393 105.3288) (width 0.2) (layer "F.Cu") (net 7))
 (segment (start 73.4347 88.7256) (end 73.4347 89.6273) (width 0.2) (layer "F.Cu") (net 7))
 (segment (start 62.0806 112.1042) (end 59.8086 114.3762) (width 0.2) (layer "F.Cu") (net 7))
 (segment (start 73.393 105.3288) (end 73.393 104.878) (width 0.2) (layer "F.Cu") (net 7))
 (segment (start 73.393 105.6699) (end 66.9587 112.1042) (width 0.2) (layer "F.Cu") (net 7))
 (segment (start 73.393 105.3288) (end 73.393 105.6699) (width 0.2) (layer "F.Cu") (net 7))
 (via (at 59.8086 114.3762) (size 0.6) (drill 0.3) (layers "F.Cu" "B.Cu") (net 7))
 (segment (start 59.8086 114.3762) (end 59.8086 127.0469) (width 0.2) (layer "B.Cu") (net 7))
 (segment (start 59.8086 127.0469) (end 61.66 128.8983) (width 0.2) (layer "B.Cu") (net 7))
 (segment (start 61.66 130) (end 61.66 128.8983) (width 0.2) (layer "B.Cu") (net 7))
 (segment (start 63.798 86.7882) (end 67.7956 86.7882) (width 0.2) (layer "F.Cu") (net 10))
 (segment (start 67.7956 86.7882) (end 69.733 88.7256) (width 0.2) (layer "F.Cu") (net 10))
 (segment (start 70.6347 88.7256) (end 69.733 88.7256) (width 0.2) (layer "F.Cu") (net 10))
 (via (at 63.798 86.7882) (size 0.6) (drill 0.3) (layers "F.Cu" "B.Cu") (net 10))
 (segment (start 63.725 97.25) (end 63.725 95.6483) (width 0.2) (layer "B.Cu") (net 10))
 (segment (start 63.798 95.5753) (end 63.798 86.7882) (width 0.2) (layer "B.Cu") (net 10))
 (segment (start 63.725 95.6483) (end 63.798 95.5753) (width 0.2) (layer "B.Cu") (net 10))
 (segment (start 70.593 105.7797) (end 69.6913 105.7797) (width 0.2) (layer "F.Cu") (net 8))
 (segment (start 68.4334 104.5218) (end 69.6913 105.7797) (width 0.2) (layer "F.Cu") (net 8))
 (segment (start 63.798 104.5218) (end 68.4334 104.5218) (width 0.2) (layer "F.Cu") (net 8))
 (via (at 63.798 104.5218) (size 0.6) (drill 0.3) (layers "F.Cu" "B.Cu") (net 8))
 (segment (start 63.798 112.5753) (end 63.798 104.5218) (width 0.2) (layer "B.Cu") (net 8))
 (segment (start 63.725 114.25) (end 63.725 112.6483) (width 0.2) (layer "B.Cu") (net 8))
 (segment (start 63.725 112.6483) (end 63.798 112.5753) (width 0.2) (layer "B.Cu") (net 8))
 (segment (start 50.7433 89.7438) (end 51.7198 88.7673) (width 0.2) (layer "F.Cu") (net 14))
 (segment (start 52.6215 88.7673) (end 51.7198 88.7673) (width 0.2) (layer "F.Cu") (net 14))
 (segment (start 45.8796 89.7438) (end 50.7433 89.7438) (width 0.2) (layer "F.Cu") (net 14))
 (via (at 45.8796 89.7438) (size 0.6) (drill 0.3) (layers "F.Cu" "B.Cu") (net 14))
 (segment (start 45.8796 95.4937) (end 45.8796 89.7438) (width 0.2) (layer "B.Cu") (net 14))
 (segment (start 45.725 95.6483) (end 45.8796 95.4937) (width 0.2) (layer "B.Cu") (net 14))
 (segment (start 45.725 97.25) (end 45.725 95.6483) (width 0.2) (layer "B.Cu") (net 14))
 (segment (start 57.4034 105.9954) (end 56.5806 105.9954) (width 0.2) (layer "F.Cu") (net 1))
 (segment (start 56.5806 105.9954) (end 56.3232 105.738) (width 0.2) (layer "F.Cu") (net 1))
 (segment (start 55.4215 105.738) (end 56.3232 105.738) (width 0.2) (layer "F.Cu") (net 1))
 (segment (start 55.4215 88.7673) (end 56.549 88.7673) (width 0.2) (layer "F.Cu") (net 1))
 (via (at 57.4034 105.9954) (size 0.6) (drill 0.3) (layers "F.Cu" "B.Cu") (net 1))
 (via (at 56.549 88.7673) (size 0.6) (drill 0.3) (layers "F.Cu" "B.Cu") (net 1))
 (segment (start 58.8767 104.5221) (end 58.8767 98.025) (width 0.2) (layer "B.Cu") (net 1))
 (segment (start 57.4034 111.1201) (end 57.4034 105.9954) (width 0.2) (layer "B.Cu") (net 1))
 (segment (start 65.72 119.4367) (end 57.4034 111.1201) (width 0.2) (layer "B.Cu") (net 1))
 (segment (start 58.8767 98.025) (end 56.549 95.6973) (width 0.2) (layer "B.Cu") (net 1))
 (segment (start 65.72 130) (end 65.72 119.4367) (width 0.2) (layer "B.Cu") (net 1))
 (segment (start 56.549 95.6973) (end 56.549 88.7673) (width 0.2) (layer "B.Cu") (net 1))
 (segment (start 57.4034 105.9954) (end 58.8767 104.5221) (width 0.2) (layer "B.Cu") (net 1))
 (segment (start 49.9567 107.5011) (end 51.7198 105.738) (width 0.2) (layer "F.Cu") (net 2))
 (segment (start 52.6215 105.738) (end 51.7198 105.738) (width 0.2) (layer "F.Cu") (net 2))
 (segment (start 45.9033 107.5011) (end 49.9567 107.5011) (width 0.2) (layer "F.Cu") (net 2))
 (via (at 45.9033 107.5011) (size 0.6) (drill 0.3) (layers "F.Cu" "B.Cu") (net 2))
 (segment (start 45.9033 112.47) (end 45.9033 107.5011) (width 0.2) (layer "B.Cu") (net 2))
 (segment (start 45.725 114.25) (end 45.725 112.6483) (width 0.2) (layer "B.Cu") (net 2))
 (segment (start 45.725 112.6483) (end 45.9033 112.47) (width 0.2) (layer "B.Cu") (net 2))
 (segment (start 57.275 102.1164) (end 75.275 102.1164) (width 0.2) (layer "F.Cu") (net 13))
 (via (at 75.275 102.1164) (size 0.6) (drill 0.3) (layers "F.Cu" "B.Cu") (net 13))
 (via (at 57.275 102.1164) (size 0.6) (drill 0.3) (layers "F.Cu" "B.Cu") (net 13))
 (segment (start 56.7927 112.941) (end 56.7927 102.5987) (width 0.2) (layer "B.Cu") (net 13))
 (segment (start 58.8767 126.6016) (end 58.8767 115.025) (width 0.2) (layer "B.Cu") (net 13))
 (segment (start 56.7927 102.5987) (end 57.275 102.1164) (width 0.2) (layer "B.Cu") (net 13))
 (segment (start 57.275 99.45) (end 57.275 102.1164) (width 0.2) (layer "B.Cu") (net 13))
 (segment (start 75.275 99.45) (end 75.275 102.1164) (width 0.2) (layer "B.Cu") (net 13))
 (segment (start 56.58 128.8983) (end 58.8767 126.6016) (width 0.2) (layer "B.Cu") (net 13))
 (segment (start 58.8767 115.025) (end 56.7927 112.941) (width 0.2) (layer "B.Cu") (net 13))
 (segment (start 56.58 130) (end 56.58 128.8983) (width 0.2) (layer "B.Cu") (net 13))
 (segment (start 66.99 127.7215) (end 66.99 130.3611) (width 0.2) (layer "B.Cu") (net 9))
 (segment (start 60.2217 130.2283) (end 60.2217 130) (width 0.2) (layer "B.Cu") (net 9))
 (segment (start 66.2248 131.1263) (end 61.1197 131.1263) (width 0.2) (layer "B.Cu") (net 9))
 (segment (start 55.444 130.4349) (end 55.444 119.8827) (width 0.2) (layer "B.Cu") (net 9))
 (segment (start 58.0183 130) (end 58.0183 130.1377) (width 0.2) (layer "B.Cu") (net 9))
 (segment (start 57.275 116.45) (end 57.275 118.0517) (width 0.2) (layer "B.Cu") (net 9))
 (segment (start 57.0013 131.1547) (end 56.1638 131.1547) (width 0.2) (layer "B.Cu") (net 9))
 (segment (start 58.0183 130.1377) (end 57.0013 131.1547) (width 0.2) (layer "B.Cu") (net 9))
 (segment (start 59.3643 130) (end 60.2217 130) (width 0.2) (layer "B.Cu") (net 9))
 (segment (start 75.275 116.45) (end 75.275 119.4365) (width 0.2) (layer "B.Cu") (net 9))
 (segment (start 75.275 119.4365) (end 66.99 127.7215) (width 0.2) (layer "B.Cu") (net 9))
 (segment (start 66.99 130.3611) (end 66.2248 131.1263) (width 0.2) (layer "B.Cu") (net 9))
 (segment (start 59.3643 130) (end 59.12 130) (width 0.2) (layer "B.Cu") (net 9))
 (segment (start 55.444 119.8827) (end 57.275 118.0517) (width 0.2) (layer "B.Cu") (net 9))
 (segment (start 56.1638 131.1547) (end 55.444 130.4349) (width 0.2) (layer "B.Cu") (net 9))
 (segment (start 59.12 130) (end 58.0183 130) (width 0.2) (layer "B.Cu") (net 9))
 (segment (start 61.1197 131.1263) (end 60.2217 130.2283) (width 0.2) (layer "B.Cu") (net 9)))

